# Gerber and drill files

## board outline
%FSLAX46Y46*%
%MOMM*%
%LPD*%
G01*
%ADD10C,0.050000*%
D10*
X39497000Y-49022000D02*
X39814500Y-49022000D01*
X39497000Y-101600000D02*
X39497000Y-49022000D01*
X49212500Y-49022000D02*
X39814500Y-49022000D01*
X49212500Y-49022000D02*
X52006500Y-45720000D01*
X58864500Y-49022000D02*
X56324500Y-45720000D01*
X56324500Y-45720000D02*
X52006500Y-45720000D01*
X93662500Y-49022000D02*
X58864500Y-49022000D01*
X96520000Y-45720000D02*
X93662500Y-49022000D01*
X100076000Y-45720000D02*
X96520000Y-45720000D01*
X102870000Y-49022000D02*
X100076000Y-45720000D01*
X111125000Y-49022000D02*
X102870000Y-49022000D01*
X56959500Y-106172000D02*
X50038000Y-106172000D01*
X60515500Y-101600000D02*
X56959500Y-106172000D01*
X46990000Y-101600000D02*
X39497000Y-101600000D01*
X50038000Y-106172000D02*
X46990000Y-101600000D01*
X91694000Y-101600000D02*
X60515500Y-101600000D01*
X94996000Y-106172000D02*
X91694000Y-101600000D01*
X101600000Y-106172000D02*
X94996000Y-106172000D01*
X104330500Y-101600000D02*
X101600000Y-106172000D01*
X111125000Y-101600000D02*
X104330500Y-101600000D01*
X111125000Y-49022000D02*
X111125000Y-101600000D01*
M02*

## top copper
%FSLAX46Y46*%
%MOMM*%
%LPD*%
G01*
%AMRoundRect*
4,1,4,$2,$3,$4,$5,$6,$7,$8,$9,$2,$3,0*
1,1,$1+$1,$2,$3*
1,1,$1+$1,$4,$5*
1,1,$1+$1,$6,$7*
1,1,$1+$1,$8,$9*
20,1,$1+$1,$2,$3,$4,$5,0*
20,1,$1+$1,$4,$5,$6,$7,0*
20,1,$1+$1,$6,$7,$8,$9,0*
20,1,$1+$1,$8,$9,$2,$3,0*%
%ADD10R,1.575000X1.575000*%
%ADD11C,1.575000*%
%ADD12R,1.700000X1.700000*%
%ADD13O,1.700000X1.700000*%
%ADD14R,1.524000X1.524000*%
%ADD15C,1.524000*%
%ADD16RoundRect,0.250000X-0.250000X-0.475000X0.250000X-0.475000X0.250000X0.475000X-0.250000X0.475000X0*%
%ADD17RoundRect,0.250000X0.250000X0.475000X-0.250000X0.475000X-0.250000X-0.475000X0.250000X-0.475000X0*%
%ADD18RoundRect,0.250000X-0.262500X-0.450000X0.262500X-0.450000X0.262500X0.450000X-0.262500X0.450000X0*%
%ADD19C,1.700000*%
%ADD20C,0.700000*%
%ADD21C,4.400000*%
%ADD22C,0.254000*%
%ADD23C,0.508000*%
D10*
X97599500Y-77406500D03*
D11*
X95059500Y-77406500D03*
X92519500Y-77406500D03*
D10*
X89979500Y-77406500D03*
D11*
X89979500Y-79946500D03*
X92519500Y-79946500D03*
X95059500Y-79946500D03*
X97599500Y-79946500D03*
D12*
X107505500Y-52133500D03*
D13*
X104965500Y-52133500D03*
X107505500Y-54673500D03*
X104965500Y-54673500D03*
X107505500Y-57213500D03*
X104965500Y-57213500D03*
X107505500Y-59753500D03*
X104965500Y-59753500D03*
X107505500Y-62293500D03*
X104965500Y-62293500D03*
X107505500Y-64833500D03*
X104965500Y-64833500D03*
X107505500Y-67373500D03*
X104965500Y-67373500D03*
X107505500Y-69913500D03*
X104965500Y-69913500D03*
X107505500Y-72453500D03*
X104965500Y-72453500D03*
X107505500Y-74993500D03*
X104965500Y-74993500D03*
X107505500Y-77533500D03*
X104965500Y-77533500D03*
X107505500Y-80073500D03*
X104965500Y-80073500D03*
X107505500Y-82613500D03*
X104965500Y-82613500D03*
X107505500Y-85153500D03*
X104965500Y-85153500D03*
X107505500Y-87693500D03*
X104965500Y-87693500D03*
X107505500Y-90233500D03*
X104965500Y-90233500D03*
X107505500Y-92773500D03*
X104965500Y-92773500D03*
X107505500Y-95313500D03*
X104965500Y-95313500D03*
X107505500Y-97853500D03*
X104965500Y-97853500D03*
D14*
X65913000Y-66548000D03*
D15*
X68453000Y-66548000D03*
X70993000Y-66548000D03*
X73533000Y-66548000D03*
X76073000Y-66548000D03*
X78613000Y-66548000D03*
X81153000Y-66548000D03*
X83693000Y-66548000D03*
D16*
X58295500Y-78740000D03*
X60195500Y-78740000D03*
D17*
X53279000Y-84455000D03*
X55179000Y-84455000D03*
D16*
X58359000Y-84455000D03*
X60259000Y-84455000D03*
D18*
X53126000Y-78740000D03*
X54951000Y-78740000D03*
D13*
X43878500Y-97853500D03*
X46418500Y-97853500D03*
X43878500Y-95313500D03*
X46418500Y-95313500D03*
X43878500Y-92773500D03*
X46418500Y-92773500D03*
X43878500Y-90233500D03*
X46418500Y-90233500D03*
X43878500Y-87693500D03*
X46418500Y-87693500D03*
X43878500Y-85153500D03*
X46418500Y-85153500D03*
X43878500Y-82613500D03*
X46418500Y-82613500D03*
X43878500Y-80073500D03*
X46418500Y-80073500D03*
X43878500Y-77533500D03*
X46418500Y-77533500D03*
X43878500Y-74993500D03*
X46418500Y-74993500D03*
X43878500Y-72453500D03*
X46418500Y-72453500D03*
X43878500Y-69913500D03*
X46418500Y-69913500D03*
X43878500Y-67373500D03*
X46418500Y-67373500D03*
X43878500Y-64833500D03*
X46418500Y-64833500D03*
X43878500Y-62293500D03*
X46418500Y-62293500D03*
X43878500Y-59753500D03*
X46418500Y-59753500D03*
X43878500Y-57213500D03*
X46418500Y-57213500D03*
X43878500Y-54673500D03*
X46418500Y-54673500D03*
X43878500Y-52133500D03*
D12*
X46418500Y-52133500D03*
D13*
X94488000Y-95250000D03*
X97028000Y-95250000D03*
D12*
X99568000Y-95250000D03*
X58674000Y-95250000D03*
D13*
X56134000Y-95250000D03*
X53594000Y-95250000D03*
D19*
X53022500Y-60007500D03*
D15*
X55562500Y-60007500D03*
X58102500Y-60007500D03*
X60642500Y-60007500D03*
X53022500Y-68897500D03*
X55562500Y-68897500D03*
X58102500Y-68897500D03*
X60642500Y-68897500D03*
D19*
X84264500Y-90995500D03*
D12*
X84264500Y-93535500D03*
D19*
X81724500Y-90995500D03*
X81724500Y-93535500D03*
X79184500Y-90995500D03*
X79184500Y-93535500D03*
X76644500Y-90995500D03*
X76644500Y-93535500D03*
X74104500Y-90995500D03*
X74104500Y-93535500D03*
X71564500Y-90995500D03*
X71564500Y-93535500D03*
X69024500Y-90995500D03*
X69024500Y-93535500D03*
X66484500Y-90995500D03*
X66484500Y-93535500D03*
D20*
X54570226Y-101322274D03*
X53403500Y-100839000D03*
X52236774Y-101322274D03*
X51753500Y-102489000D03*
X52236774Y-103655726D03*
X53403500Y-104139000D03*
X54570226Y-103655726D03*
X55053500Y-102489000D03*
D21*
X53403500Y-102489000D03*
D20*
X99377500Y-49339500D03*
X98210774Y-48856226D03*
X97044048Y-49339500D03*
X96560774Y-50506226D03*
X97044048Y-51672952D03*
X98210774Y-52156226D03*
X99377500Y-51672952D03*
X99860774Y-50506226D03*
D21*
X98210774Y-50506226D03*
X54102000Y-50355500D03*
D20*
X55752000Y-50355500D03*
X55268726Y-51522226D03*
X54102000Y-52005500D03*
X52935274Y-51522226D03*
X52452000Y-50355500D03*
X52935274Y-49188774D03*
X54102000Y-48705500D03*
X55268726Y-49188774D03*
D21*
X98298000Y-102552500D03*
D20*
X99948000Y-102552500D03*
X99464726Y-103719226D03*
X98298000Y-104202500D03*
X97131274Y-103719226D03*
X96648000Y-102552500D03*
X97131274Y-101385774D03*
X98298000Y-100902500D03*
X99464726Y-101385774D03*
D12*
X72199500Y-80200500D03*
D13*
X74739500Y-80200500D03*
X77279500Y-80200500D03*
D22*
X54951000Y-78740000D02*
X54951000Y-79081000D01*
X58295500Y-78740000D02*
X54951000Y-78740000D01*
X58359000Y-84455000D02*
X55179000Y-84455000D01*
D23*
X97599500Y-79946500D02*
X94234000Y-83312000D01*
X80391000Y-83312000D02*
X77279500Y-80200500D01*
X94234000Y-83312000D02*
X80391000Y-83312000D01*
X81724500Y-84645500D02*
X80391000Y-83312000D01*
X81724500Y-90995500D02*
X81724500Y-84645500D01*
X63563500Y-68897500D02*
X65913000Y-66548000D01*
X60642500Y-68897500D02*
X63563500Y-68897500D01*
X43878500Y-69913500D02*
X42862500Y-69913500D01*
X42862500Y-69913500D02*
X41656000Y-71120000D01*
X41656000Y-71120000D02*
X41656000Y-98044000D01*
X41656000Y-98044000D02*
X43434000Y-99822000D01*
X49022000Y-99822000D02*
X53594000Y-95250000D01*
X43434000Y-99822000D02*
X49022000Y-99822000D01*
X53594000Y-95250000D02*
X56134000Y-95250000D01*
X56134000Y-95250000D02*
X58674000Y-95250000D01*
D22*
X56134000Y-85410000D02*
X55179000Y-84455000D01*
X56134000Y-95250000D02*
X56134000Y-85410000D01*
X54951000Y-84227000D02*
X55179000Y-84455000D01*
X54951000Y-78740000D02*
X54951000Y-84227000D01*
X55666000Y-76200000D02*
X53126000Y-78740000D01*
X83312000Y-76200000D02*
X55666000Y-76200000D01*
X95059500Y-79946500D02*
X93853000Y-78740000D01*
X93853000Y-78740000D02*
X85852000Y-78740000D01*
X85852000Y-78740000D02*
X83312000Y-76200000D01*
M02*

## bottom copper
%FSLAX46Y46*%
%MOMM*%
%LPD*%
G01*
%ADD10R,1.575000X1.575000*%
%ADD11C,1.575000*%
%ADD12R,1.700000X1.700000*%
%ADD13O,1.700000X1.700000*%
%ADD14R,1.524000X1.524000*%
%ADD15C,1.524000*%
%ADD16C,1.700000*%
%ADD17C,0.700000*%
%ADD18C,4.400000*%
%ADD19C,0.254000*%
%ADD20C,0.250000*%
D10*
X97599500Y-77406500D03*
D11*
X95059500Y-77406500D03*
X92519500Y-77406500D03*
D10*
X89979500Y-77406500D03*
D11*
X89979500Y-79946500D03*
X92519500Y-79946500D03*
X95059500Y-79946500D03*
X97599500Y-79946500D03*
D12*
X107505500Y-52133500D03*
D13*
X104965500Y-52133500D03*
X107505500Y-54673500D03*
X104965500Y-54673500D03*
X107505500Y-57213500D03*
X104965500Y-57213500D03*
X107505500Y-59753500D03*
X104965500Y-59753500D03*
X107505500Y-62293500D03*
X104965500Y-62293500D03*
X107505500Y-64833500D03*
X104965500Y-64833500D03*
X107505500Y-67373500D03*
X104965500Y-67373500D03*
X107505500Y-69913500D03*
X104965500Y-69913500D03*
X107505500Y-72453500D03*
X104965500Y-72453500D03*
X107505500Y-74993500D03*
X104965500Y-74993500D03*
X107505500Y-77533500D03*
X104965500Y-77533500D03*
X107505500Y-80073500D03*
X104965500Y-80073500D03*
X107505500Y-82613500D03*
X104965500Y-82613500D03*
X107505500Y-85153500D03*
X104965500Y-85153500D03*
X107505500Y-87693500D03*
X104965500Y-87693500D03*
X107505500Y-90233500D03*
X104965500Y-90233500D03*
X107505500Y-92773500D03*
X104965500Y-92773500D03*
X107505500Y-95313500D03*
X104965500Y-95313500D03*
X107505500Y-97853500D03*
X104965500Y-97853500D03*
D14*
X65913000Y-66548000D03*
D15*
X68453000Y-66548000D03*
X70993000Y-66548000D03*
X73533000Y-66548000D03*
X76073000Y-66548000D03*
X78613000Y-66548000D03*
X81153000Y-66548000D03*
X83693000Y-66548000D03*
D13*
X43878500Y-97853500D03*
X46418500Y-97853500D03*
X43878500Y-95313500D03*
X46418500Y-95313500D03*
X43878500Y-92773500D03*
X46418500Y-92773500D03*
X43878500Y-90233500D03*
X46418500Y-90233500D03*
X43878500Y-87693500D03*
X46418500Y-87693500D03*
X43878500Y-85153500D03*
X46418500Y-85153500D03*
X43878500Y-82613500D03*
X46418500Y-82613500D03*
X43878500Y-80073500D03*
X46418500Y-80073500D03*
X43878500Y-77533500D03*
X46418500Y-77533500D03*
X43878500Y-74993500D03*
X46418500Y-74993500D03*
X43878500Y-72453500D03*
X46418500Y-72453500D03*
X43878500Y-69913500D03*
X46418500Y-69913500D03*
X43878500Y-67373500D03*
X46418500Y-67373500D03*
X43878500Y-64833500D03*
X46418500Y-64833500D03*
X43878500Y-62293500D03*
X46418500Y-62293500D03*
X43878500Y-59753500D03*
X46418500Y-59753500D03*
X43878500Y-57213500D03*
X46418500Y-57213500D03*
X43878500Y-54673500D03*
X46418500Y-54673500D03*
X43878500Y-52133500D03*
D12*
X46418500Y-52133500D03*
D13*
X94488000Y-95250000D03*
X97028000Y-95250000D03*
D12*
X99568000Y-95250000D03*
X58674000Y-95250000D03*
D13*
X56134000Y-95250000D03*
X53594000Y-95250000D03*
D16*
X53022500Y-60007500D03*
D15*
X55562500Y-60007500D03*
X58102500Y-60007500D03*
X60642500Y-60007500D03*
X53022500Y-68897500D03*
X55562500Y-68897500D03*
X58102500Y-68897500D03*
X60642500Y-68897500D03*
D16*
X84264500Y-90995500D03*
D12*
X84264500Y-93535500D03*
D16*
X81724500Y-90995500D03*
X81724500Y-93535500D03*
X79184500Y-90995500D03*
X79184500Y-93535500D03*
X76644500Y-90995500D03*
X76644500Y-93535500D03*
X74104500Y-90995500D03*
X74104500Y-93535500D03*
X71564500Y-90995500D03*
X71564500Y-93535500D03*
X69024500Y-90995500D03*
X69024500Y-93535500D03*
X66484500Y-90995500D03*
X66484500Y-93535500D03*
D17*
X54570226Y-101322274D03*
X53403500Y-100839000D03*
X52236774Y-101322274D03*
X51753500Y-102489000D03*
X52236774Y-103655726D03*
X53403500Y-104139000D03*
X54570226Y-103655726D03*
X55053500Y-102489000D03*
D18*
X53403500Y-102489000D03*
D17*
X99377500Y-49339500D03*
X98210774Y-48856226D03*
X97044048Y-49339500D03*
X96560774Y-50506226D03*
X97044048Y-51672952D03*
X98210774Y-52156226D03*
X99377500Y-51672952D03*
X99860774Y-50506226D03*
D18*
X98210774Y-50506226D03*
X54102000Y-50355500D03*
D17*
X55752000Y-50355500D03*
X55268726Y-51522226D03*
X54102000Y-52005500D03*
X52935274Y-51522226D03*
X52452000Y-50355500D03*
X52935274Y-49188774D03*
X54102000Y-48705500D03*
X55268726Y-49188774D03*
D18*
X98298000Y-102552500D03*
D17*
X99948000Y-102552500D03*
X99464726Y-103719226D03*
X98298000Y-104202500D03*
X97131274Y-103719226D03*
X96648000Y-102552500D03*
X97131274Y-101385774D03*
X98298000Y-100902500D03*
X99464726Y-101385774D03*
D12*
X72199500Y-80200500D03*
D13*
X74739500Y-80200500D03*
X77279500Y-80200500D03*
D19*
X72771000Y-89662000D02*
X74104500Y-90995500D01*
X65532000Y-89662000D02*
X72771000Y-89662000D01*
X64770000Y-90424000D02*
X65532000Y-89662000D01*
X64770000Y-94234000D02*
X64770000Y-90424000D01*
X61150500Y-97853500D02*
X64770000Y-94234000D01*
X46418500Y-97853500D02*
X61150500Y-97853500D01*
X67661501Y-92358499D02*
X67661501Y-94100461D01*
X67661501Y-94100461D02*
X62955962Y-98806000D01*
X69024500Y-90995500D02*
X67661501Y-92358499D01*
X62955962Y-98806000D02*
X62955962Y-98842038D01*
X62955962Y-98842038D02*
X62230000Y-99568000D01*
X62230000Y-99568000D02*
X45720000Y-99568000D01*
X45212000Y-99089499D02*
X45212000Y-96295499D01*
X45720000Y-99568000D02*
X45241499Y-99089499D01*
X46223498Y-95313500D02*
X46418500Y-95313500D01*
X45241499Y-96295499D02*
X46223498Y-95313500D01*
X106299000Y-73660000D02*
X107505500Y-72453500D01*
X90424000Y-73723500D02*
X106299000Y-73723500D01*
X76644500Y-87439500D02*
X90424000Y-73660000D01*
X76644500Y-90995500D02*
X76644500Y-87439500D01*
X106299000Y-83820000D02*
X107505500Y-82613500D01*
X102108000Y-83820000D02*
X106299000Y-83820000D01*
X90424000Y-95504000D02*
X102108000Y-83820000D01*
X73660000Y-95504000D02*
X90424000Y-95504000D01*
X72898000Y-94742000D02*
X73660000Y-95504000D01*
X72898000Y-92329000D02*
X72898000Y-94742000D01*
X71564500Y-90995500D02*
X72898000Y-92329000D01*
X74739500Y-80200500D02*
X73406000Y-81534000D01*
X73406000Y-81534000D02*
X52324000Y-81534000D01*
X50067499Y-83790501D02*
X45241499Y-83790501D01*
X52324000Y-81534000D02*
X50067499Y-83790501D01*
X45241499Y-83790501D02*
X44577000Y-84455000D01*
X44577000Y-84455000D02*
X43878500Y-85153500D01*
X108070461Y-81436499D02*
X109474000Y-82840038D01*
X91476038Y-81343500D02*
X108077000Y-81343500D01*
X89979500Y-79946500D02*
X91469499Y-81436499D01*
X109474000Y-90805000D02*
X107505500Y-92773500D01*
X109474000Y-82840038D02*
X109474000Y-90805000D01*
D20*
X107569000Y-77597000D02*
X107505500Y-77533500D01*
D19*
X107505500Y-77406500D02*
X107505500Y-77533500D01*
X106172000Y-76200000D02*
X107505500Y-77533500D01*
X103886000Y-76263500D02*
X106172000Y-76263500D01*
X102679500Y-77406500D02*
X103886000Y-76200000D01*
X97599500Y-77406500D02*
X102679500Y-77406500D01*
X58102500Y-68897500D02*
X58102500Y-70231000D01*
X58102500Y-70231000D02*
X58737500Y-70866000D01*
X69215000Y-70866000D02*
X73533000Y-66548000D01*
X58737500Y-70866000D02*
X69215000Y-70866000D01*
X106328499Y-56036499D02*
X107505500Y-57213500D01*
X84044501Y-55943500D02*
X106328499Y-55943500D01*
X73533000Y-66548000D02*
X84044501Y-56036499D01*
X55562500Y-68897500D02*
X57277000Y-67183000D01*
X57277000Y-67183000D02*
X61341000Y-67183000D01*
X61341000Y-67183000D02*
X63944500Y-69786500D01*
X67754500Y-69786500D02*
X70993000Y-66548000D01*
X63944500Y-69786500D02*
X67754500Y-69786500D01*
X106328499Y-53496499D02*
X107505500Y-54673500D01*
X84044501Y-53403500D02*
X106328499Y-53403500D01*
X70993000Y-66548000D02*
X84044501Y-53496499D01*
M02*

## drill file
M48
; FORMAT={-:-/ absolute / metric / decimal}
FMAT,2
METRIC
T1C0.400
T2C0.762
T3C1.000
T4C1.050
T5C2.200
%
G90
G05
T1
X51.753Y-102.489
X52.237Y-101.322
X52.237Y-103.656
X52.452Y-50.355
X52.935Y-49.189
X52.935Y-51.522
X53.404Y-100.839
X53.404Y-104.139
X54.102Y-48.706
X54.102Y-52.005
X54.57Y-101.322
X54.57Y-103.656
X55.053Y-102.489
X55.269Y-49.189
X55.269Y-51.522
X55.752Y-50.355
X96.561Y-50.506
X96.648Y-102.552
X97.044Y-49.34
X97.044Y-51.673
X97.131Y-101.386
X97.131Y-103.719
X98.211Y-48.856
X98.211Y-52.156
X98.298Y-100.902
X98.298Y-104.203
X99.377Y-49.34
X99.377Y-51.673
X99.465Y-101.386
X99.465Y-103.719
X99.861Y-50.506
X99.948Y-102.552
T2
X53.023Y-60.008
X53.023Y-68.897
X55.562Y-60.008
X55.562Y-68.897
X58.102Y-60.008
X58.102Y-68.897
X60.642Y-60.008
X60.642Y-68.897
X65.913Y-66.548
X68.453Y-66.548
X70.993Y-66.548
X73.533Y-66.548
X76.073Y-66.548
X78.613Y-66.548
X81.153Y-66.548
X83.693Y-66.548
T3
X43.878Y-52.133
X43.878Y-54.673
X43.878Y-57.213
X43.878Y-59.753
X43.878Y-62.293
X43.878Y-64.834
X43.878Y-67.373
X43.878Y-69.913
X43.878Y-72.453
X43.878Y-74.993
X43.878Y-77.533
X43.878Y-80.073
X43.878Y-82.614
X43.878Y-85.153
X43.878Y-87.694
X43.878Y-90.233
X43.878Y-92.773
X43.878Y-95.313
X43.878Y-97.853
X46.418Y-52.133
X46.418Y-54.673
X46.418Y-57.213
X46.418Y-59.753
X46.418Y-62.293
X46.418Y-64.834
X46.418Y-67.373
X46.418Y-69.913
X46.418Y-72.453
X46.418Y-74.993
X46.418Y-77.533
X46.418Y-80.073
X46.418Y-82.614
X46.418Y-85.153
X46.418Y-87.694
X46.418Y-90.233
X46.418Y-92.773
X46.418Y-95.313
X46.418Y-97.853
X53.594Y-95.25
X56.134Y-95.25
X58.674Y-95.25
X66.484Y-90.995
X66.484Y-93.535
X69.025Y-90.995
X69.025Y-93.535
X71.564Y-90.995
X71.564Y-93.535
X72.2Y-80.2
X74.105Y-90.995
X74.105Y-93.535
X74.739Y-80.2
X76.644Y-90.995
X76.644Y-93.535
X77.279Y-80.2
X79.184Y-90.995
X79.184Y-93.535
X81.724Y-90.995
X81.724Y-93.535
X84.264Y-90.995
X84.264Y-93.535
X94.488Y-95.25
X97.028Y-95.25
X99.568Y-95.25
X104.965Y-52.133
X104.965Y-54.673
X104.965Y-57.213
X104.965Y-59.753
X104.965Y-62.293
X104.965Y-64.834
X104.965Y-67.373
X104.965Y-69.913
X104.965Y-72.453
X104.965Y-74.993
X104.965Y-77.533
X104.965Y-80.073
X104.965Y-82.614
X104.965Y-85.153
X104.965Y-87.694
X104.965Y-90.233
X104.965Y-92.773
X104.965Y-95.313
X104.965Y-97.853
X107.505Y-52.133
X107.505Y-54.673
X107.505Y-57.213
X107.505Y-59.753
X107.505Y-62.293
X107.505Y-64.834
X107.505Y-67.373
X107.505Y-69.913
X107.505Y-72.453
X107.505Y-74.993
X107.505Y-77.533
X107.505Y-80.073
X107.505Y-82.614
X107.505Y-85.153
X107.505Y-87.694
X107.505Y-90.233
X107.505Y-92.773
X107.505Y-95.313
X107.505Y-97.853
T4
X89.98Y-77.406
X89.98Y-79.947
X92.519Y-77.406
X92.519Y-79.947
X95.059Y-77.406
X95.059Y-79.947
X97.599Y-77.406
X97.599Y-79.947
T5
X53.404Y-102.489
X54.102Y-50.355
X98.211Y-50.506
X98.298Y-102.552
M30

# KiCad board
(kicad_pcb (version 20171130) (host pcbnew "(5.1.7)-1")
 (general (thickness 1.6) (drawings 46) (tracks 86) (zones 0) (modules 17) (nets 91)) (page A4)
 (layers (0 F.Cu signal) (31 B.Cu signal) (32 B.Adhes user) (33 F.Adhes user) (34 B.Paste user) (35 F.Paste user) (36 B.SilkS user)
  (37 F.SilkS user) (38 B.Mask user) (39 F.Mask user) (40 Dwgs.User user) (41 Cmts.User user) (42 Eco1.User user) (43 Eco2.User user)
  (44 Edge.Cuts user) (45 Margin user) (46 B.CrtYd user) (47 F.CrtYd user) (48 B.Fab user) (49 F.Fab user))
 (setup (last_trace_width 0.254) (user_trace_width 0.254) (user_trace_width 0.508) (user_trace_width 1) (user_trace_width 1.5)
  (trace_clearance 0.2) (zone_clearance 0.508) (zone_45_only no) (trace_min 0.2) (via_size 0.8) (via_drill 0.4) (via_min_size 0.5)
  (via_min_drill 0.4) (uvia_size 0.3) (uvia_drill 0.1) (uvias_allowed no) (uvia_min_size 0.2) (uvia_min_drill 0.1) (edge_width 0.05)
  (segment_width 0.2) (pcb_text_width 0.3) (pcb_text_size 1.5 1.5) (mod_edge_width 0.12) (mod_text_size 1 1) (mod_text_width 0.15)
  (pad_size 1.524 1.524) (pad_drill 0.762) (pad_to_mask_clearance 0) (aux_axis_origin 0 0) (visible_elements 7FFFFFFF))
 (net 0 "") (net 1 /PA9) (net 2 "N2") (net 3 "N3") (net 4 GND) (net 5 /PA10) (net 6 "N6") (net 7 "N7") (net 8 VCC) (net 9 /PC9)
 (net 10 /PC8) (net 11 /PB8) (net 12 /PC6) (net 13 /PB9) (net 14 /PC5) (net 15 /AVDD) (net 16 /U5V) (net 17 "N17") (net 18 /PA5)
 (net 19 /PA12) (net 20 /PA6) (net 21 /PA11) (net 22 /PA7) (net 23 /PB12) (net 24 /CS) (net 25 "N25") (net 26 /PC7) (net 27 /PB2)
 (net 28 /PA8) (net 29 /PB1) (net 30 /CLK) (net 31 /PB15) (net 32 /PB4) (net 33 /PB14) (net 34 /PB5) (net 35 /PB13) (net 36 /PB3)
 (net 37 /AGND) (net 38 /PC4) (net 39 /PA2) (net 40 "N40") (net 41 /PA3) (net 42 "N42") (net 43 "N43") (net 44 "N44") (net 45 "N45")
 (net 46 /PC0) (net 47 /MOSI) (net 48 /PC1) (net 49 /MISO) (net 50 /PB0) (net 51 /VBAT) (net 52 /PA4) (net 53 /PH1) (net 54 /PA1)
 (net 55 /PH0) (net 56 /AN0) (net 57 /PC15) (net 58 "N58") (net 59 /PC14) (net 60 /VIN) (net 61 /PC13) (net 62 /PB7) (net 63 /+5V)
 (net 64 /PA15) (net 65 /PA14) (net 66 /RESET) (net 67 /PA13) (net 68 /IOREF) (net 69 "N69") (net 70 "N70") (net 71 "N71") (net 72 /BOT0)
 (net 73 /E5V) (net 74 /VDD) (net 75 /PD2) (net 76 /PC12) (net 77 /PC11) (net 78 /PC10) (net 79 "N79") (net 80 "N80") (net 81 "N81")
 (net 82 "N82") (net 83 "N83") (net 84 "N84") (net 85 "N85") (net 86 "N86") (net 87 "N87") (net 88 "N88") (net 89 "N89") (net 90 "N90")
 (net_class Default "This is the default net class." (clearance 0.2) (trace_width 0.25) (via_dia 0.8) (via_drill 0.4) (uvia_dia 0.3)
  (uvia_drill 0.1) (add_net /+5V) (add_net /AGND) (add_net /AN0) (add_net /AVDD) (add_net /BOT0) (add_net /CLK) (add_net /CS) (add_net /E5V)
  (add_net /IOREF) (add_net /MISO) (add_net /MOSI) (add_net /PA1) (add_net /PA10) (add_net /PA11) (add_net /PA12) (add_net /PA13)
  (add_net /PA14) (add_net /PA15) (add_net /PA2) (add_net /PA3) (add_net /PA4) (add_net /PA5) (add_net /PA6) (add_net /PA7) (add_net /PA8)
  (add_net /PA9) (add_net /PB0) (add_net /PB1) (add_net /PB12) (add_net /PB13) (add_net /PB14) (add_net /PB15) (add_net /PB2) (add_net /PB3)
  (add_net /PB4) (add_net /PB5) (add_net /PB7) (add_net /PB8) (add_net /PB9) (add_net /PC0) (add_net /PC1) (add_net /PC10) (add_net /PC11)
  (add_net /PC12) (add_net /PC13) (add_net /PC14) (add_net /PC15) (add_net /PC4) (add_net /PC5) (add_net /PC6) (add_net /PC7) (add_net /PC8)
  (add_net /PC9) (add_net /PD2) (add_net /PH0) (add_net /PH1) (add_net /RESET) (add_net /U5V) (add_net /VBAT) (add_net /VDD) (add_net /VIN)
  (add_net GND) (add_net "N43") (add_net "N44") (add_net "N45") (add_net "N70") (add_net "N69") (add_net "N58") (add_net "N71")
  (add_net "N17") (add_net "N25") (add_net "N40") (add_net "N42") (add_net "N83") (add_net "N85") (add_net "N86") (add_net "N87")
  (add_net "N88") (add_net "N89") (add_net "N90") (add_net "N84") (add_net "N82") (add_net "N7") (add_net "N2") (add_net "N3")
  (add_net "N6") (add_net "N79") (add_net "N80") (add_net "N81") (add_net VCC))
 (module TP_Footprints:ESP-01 (layer F.Cu) (at 93.7895 77.4065 90)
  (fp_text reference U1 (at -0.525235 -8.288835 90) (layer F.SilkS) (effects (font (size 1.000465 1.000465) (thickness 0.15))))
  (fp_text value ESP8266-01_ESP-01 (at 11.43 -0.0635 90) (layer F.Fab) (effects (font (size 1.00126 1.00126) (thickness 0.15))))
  (pad 1 thru_hole rect (at 0 3.81 90) (size 1.575 1.575) (drill 1.05) (layers *.Cu *.Mask) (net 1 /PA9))
  (pad 2 thru_hole circle (at 0 1.27 90) (size 1.575 1.575) (drill 1.05) (layers *.Cu *.Mask) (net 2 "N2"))
  (pad 3 thru_hole circle (at 0 -1.27 90) (size 1.575 1.575) (drill 1.05) (layers *.Cu *.Mask) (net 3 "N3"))
  (pad 4 thru_hole rect (at 0 -3.81 90) (size 1.575 1.575) (drill 1.05) (layers *.Cu *.Mask) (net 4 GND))
  (pad 5 thru_hole circle (at -2.54 -3.81 90) (size 1.575 1.575) (drill 1.05) (layers *.Cu *.Mask) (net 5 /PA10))
  (pad 6 thru_hole circle (at -2.54 -1.27 90) (size 1.575 1.575) (drill 1.05) (layers *.Cu *.Mask) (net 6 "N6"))
  (pad 7 thru_hole circle (at -2.54 1.27 90) (size 1.575 1.575) (drill 1.05) (layers *.Cu *.Mask) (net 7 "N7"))
  (pad 8 thru_hole circle (at -2.54 3.81 90) (size 1.575 1.575) (drill 1.05) (layers *.Cu *.Mask) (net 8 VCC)))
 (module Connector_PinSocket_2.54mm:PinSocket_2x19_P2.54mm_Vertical (layer F.Cu) (at 107.5055 52.1335)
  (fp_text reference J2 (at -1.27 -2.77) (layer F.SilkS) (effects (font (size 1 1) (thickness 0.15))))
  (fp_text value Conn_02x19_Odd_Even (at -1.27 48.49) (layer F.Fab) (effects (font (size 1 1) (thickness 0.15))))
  (pad 1 thru_hole rect (at 0 0) (size 1.7 1.7) (drill 1) (layers *.Cu *.Mask) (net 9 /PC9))
  (pad 2 thru_hole oval (at -2.54 0) (size 1.7 1.7) (drill 1) (layers *.Cu *.Mask) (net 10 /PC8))
  (pad 3 thru_hole oval (at 0 2.54) (size 1.7 1.7) (drill 1) (layers *.Cu *.Mask) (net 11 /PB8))
  (pad 4 thru_hole oval (at -2.54 2.54) (size 1.7 1.7) (drill 1) (layers *.Cu *.Mask) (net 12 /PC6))
  (pad 5 thru_hole oval (at 0 5.08) (size 1.7 1.7) (drill 1) (layers *.Cu *.Mask) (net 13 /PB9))
  (pad 6 thru_hole oval (at -2.54 5.08) (size 1.7 1.7) (drill 1) (layers *.Cu *.Mask) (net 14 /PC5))
  (pad 7 thru_hole oval (at 0 7.62) (size 1.7 1.7) (drill 1) (layers *.Cu *.Mask) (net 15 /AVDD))
  (pad 8 thru_hole oval (at -2.54 7.62) (size 1.7 1.7) (drill 1) (layers *.Cu *.Mask) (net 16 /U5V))
  (pad 9 thru_hole oval (at 0 10.16) (size 1.7 1.7) (drill 1) (layers *.Cu *.Mask) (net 4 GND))
  (pad 10 thru_hole oval (at -2.54 10.16) (size 1.7 1.7) (drill 1) (layers *.Cu *.Mask) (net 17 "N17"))
  (pad 11 thru_hole oval (at 0 12.7) (size 1.7 1.7) (drill 1) (layers *.Cu *.Mask) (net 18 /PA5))
  (pad 12 thru_hole oval (at -2.54 12.7) (size 1.7 1.7) (drill 1) (layers *.Cu *.Mask) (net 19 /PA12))
  (pad 13 thru_hole oval (at 0 15.24) (size 1.7 1.7) (drill 1) (layers *.Cu *.Mask) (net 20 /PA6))
  (pad 14 thru_hole oval (at -2.54 15.24) (size 1.7 1.7) (drill 1) (layers *.Cu *.Mask) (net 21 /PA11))
  (pad 15 thru_hole oval (at 0 17.78) (size 1.7 1.7) (drill 1) (layers *.Cu *.Mask) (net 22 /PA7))
  (pad 16 thru_hole oval (at -2.54 17.78) (size 1.7 1.7) (drill 1) (layers *.Cu *.Mask) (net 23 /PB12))
  (pad 17 thru_hole oval (at 0 20.32) (size 1.7 1.7) (drill 1) (layers *.Cu *.Mask) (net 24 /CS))
  (pad 18 thru_hole oval (at -2.54 20.32) (size 1.7 1.7) (drill 1) (layers *.Cu *.Mask) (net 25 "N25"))
  (pad 19 thru_hole oval (at 0 22.86) (size 1.7 1.7) (drill 1) (layers *.Cu *.Mask) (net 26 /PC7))
  (pad 20 thru_hole oval (at -2.54 22.86) (size 1.7 1.7) (drill 1) (layers *.Cu *.Mask) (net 4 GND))
  (pad 21 thru_hole oval (at 0 25.4) (size 1.7 1.7) (drill 1) (layers *.Cu *.Mask) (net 1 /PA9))
  (pad 22 thru_hole oval (at -2.54 25.4) (size 1.7 1.7) (drill 1) (layers *.Cu *.Mask) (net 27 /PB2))
  (pad 23 thru_hole oval (at 0 27.94) (size 1.7 1.7) (drill 1) (layers *.Cu *.Mask) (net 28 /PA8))
  (pad 24 thru_hole oval (at -2.54 27.94) (size 1.7 1.7) (drill 1) (layers *.Cu *.Mask) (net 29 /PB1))
  (pad 25 thru_hole oval (at 0 30.48) (size 1.7 1.7) (drill 1) (layers *.Cu *.Mask) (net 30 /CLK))
  (pad 26 thru_hole oval (at -2.54 30.48) (size 1.7 1.7) (drill 1) (layers *.Cu *.Mask) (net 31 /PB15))
  (pad 27 thru_hole oval (at 0 33.02) (size 1.7 1.7) (drill 1) (layers *.Cu *.Mask) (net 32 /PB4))
  (pad 28 thru_hole oval (at -2.54 33.02) (size 1.7 1.7) (drill 1) (layers *.Cu *.Mask) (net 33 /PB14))
  (pad 29 thru_hole oval (at 0 35.56) (size 1.7 1.7) (drill 1) (layers *.Cu *.Mask) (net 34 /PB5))
  (pad 30 thru_hole oval (at -2.54 35.56) (size 1.7 1.7) (drill 1) (layers *.Cu *.Mask) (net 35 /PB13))
  (pad 31 thru_hole oval (at 0 38.1) (size 1.7 1.7) (drill 1) (layers *.Cu *.Mask) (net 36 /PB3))
  (pad 32 thru_hole oval (at -2.54 38.1) (size 1.7 1.7) (drill 1) (layers *.Cu *.Mask) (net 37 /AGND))
  (pad 33 thru_hole oval (at 0 40.64) (size 1.7 1.7) (drill 1) (layers *.Cu *.Mask) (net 5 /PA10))
  (pad 34 thru_hole oval (at -2.54 40.64) (size 1.7 1.7) (drill 1) (layers *.Cu *.Mask) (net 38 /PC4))
  (pad 35 thru_hole oval (at 0 43.18) (size 1.7 1.7) (drill 1) (layers *.Cu *.Mask) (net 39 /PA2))
  (pad 36 thru_hole oval (at -2.54 43.18) (size 1.7 1.7) (drill 1) (layers *.Cu *.Mask) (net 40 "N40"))
  (pad 37 thru_hole oval (at 0 45.72) (size 1.7 1.7) (drill 1) (layers *.Cu *.Mask) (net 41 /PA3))
  (pad 38 thru_hole oval (at -2.54 45.72) (size 1.7 1.7) (drill 1) (layers *.Cu *.Mask) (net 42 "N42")))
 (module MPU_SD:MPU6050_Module (layer F.Cu) (at 65.913 66.548 90)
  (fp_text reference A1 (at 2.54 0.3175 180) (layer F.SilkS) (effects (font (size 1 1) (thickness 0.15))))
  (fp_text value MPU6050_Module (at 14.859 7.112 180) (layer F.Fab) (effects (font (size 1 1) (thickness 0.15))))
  (pad 1 thru_hole rect (at 0 0 90) (size 1.524 1.524) (drill 0.762) (layers *.Cu *.Mask) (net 8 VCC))
  (pad 2 thru_hole circle (at 0 2.54 90) (size 1.524 1.524) (drill 0.762) (layers *.Cu *.Mask) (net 4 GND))
  (pad 3 thru_hole circle (at 0 5.08 90) (size 1.524 1.524) (drill 0.762) (layers *.Cu *.Mask) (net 11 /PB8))
  (pad 4 thru_hole circle (at 0 7.62 90) (size 1.524 1.524) (drill 0.762) (layers *.Cu *.Mask) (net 13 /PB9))
  (pad 5 thru_hole circle (at 0 10.16 90) (size 1.524 1.524) (drill 0.762) (layers *.Cu *.Mask) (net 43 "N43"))
  (pad 6 thru_hole circle (at 0 12.7 90) (size 1.524 1.524) (drill 0.762) (layers *.Cu *.Mask) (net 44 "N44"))
  (pad 7 thru_hole circle (at 0 15.24 90) (size 1.524 1.524) (drill 0.762) (layers *.Cu *.Mask) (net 4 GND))
  (pad 8 thru_hole circle (at 0 17.78 90) (size 1.524 1.524) (drill 0.762) (layers *.Cu *.Mask) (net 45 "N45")))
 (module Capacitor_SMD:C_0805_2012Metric (layer F.Cu) (at 59.2455 78.74)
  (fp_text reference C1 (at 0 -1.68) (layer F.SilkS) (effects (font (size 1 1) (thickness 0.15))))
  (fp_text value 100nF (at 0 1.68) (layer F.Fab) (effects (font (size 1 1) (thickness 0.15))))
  (pad 1 smd roundrect (at -0.95 0) (size 1 1.45) (layers F.Cu F.Paste F.Mask) (roundrect_rratio 0.25) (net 8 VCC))
  (pad 2 smd roundrect (at 0.95 0) (size 1 1.45) (layers F.Cu F.Paste F.Mask) (roundrect_rratio 0.25) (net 4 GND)))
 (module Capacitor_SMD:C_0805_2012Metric (layer F.Cu) (at 54.229 84.455 180)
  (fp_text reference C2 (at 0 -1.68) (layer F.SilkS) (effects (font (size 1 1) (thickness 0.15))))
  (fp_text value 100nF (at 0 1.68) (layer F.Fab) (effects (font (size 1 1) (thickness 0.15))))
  (pad 2 smd roundrect (at 0.95 0 180) (size 1 1.45) (layers F.Cu F.Paste F.Mask) (roundrect_rratio 0.25) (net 4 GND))
  (pad 1 smd roundrect (at -0.95 0 180) (size 1 1.45) (layers F.Cu F.Paste F.Mask) (roundrect_rratio 0.25) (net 8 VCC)))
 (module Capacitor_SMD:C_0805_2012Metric (layer F.Cu) (at 59.309 84.455)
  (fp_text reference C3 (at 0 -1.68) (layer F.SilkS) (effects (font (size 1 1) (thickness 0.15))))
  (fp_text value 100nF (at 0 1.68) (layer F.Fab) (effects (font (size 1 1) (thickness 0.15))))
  (pad 1 smd roundrect (at -0.95 0) (size 1 1.45) (layers F.Cu F.Paste F.Mask) (roundrect_rratio 0.25) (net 8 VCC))
  (pad 2 smd roundrect (at 0.95 0) (size 1 1.45) (layers F.Cu F.Paste F.Mask) (roundrect_rratio 0.25) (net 4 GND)))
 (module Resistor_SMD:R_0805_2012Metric (layer F.Cu) (at 54.0385 78.74)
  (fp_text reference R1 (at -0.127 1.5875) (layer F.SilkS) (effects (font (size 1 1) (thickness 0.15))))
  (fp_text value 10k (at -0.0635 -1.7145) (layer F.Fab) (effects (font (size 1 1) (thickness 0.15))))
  (pad 1 smd roundrect (at -0.9125 0) (size 1.025 1.4) (layers F.Cu F.Paste F.Mask) (roundrect_rratio 0.243902) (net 7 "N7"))
  (pad 2 smd roundrect (at 0.9125 0) (size 1.025 1.4) (layers F.Cu F.Paste F.Mask) (roundrect_rratio 0.243902) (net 8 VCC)))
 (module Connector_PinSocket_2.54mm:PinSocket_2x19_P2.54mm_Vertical (layer F.Cu) (at 46.4185 52.1335)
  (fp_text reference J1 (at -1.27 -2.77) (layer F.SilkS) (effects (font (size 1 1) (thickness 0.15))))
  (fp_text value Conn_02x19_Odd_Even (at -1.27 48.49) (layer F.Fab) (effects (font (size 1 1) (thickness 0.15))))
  (pad 38 thru_hole oval (at -2.54 45.72) (size 1.7 1.7) (drill 1) (layers *.Cu *.Mask) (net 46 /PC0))
  (pad 37 thru_hole oval (at 0 45.72) (size 1.7 1.7) (drill 1) (layers *.Cu *.Mask) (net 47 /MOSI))
  (pad 36 thru_hole oval (at -2.54 43.18) (size 1.7 1.7) (drill 1) (layers *.Cu *.Mask) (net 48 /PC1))
  (pad 35 thru_hole oval (at 0 43.18) (size 1.7 1.7) (drill 1) (layers *.Cu *.Mask) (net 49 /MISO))
  (pad 34 thru_hole oval (at -2.54 40.64) (size 1.7 1.7) (drill 1) (layers *.Cu *.Mask) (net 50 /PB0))
  (pad 33 thru_hole oval (at 0 40.64) (size 1.7 1.7) (drill 1) (layers *.Cu *.Mask) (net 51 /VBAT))
  (pad 32 thru_hole oval (at -2.54 38.1) (size 1.7 1.7) (drill 1) (layers *.Cu *.Mask) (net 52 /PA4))
  (pad 31 thru_hole oval (at 0 38.1) (size 1.7 1.7) (drill 1) (layers *.Cu *.Mask) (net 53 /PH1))
  (pad 30 thru_hole oval (at -2.54 35.56) (size 1.7 1.7) (drill 1) (layers *.Cu *.Mask) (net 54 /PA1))
  (pad 29 thru_hole oval (at 0 35.56) (size 1.7 1.7) (drill 1) (layers *.Cu *.Mask) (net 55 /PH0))
  (pad 28 thru_hole oval (at -2.54 33.02) (size 1.7 1.7) (drill 1) (layers *.Cu *.Mask) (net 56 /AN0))
  (pad 27 thru_hole oval (at 0 33.02) (size 1.7 1.7) (drill 1) (layers *.Cu *.Mask) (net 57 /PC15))
  (pad 26 thru_hole oval (at -2.54 30.48) (size 1.7 1.7) (drill 1) (layers *.Cu *.Mask) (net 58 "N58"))
  (pad 25 thru_hole oval (at 0 30.48) (size 1.7 1.7) (drill 1) (layers *.Cu *.Mask) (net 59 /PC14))
  (pad 24 thru_hole oval (at -2.54 27.94) (size 1.7 1.7) (drill 1) (layers *.Cu *.Mask) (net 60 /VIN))
  (pad 23 thru_hole oval (at 0 27.94) (size 1.7 1.7) (drill 1) (layers *.Cu *.Mask) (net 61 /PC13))
  (pad 22 thru_hole oval (at -2.54 25.4) (size 1.7 1.7) (drill 1) (layers *.Cu *.Mask) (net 4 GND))
  (pad 21 thru_hole oval (at 0 25.4) (size 1.7 1.7) (drill 1) (layers *.Cu *.Mask) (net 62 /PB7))
  (pad 20 thru_hole oval (at -2.54 22.86) (size 1.7 1.7) (drill 1) (layers *.Cu *.Mask) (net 4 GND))
  (pad 19 thru_hole oval (at 0 22.86) (size 1.7 1.7) (drill 1) (layers *.Cu *.Mask) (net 4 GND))
  (pad 18 thru_hole oval (at -2.54 20.32) (size 1.7 1.7) (drill 1) (layers *.Cu *.Mask) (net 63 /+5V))
  (pad 17 thru_hole oval (at 0 20.32) (size 1.7 1.7) (drill 1) (layers *.Cu *.Mask) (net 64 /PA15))
  (pad 16 thru_hole oval (at -2.54 17.78) (size 1.7 1.7) (drill 1) (layers *.Cu *.Mask) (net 8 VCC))
  (pad 15 thru_hole oval (at 0 17.78) (size 1.7 1.7) (drill 1) (layers *.Cu *.Mask) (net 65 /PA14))
  (pad 14 thru_hole oval (at -2.54 15.24) (size 1.7 1.7) (drill 1) (layers *.Cu *.Mask) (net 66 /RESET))
  (pad 13 thru_hole oval (at 0 15.24) (size 1.7 1.7) (drill 1) (layers *.Cu *.Mask) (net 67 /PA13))
  (pad 12 thru_hole oval (at -2.54 12.7) (size 1.7 1.7) (drill 1) (layers *.Cu *.Mask) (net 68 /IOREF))
  (pad 11 thru_hole oval (at 0 12.7) (size 1.7 1.7) (drill 1) (layers *.Cu *.Mask) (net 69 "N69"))
  (pad 10 thru_hole oval (at -2.54 10.16) (size 1.7 1.7) (drill 1) (layers *.Cu *.Mask) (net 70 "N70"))
  (pad 9 thru_hole oval (at 0 10.16) (size 1.7 1.7) (drill 1) (layers *.Cu *.Mask) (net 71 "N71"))
  (pad 8 thru_hole oval (at -2.54 7.62) (size 1.7 1.7) (drill 1) (layers *.Cu *.Mask) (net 4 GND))
  (pad 7 thru_hole oval (at 0 7.62) (size 1.7 1.7) (drill 1) (layers *.Cu *.Mask) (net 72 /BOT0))
  (pad 6 thru_hole oval (at -2.54 5.08) (size 1.7 1.7) (drill 1) (layers *.Cu *.Mask) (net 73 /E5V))
  (pad 5 thru_hole oval (at 0 5.08) (size 1.7 1.7) (drill 1) (layers *.Cu *.Mask) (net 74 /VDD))
  (pad 4 thru_hole oval (at -2.54 2.54) (size 1.7 1.7) (drill 1) (layers *.Cu *.Mask) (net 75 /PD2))
  (pad 3 thru_hole oval (at 0 2.54) (size 1.7 1.7) (drill 1) (layers *.Cu *.Mask) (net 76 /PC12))
  (pad 2 thru_hole oval (at -2.54 0) (size 1.7 1.7) (drill 1) (layers *.Cu *.Mask) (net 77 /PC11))
  (pad 1 thru_hole rect (at 0 0) (size 1.7 1.7) (drill 1) (layers *.Cu *.Mask) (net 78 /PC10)))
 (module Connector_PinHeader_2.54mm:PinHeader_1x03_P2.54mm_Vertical (layer F.Cu) (at 99.568 95.25 270)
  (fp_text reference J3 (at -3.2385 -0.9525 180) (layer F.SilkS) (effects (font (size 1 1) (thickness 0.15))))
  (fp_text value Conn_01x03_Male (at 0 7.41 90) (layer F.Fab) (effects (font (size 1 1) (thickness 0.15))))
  (pad 3 thru_hole oval (at 0 5.08 270) (size 1.7 1.7) (drill 1) (layers *.Cu *.Mask) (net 4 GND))
  (pad 2 thru_hole oval (at 0 2.54 270) (size 1.7 1.7) (drill 1) (layers *.Cu *.Mask) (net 4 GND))
  (pad 1 thru_hole rect (at 0 0 270) (size 1.7 1.7) (drill 1) (layers *.Cu *.Mask) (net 4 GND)))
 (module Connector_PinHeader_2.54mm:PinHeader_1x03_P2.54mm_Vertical (layer F.Cu) (at 58.674 95.25 270)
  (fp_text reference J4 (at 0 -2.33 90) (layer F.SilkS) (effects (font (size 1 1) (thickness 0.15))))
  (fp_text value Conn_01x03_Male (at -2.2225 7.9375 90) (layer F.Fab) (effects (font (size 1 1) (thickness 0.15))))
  (pad 1 thru_hole rect (at 0 0 270) (size 1.7 1.7) (drill 1) (layers *.Cu *.Mask) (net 8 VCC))
  (pad 2 thru_hole oval (at 0 2.54 270) (size 1.7 1.7) (drill 1) (layers *.Cu *.Mask) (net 8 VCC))
  (pad 3 thru_hole oval (at 0 5.08 270) (size 1.7 1.7) (drill 1) (layers *.Cu *.Mask) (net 8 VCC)))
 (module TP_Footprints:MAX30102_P (layer F.Cu) (at 55.5625 60.0075)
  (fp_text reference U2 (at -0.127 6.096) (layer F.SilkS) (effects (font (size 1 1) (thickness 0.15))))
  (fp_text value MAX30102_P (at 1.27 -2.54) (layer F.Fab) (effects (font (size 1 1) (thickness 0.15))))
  (pad 1 thru_hole circle (at -2.54 0) (size 1.7 1.7) (drill 0.762) (layers *.Cu *.Mask) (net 4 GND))
  (pad 2 thru_hole circle (at 0 0) (size 1.524 1.524) (drill 0.762) (layers *.Cu *.Mask) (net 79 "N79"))
  (pad 3 thru_hole circle (at 2.54 0) (size 1.524 1.524) (drill 0.762) (layers *.Cu *.Mask) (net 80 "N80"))
  (pad 4 thru_hole circle (at 5.08 0) (size 1.524 1.524) (drill 0.762) (layers *.Cu *.Mask) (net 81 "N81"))
  (pad 5 thru_hole circle (at -2.54 8.89) (size 1.524 1.524) (drill 0.762) (layers *.Cu *.Mask) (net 4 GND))
  (pad 6 thru_hole circle (at 0 8.89) (size 1.524 1.524) (drill 0.762) (layers *.Cu *.Mask) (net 11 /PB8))
  (pad 7 thru_hole circle (at 2.54 8.89) (size 1.524 1.524) (drill 0.762) (layers *.Cu *.Mask) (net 13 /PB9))
  (pad 8 thru_hole circle (at 5.08 8.89) (size 1.524 1.524) (drill 0.762) (layers *.Cu *.Mask) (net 8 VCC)))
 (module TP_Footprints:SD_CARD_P (layer F.Cu) (at 84.2645 93.5355 270)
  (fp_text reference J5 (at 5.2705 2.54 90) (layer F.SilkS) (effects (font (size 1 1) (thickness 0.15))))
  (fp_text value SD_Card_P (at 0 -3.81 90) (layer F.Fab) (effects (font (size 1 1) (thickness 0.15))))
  (pad 1 thru_hole circle (at -2.54 0 270) (size 1.7 1.7) (drill 1) (layers *.Cu *.Mask) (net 4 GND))
  (pad 9 thru_hole rect (at 0 0 270) (size 1.7 1.7) (drill 1) (layers *.Cu *.Mask) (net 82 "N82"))
  (pad 2 thru_hole circle (at -2.54 2.54 270) (size 1.7 1.7) (drill 1) (layers *.Cu *.Mask) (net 8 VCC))
  (pad 10 thru_hole circle (at 0 2.54 270) (size 1.7 1.7) (drill 1) (layers *.Cu *.Mask) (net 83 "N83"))
  (pad 3 thru_hole circle (at -2.54 5.08 270) (size 1.7 1.7) (drill 1) (layers *.Cu *.Mask) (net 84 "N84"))
  (pad 11 thru_hole circle (at 0 5.08 270) (size 1.7 1.7) (drill 1) (layers *.Cu *.Mask) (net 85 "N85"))
  (pad 4 thru_hole circle (at -2.54 7.62 270) (size 1.7 1.7) (drill 1) (layers *.Cu *.Mask) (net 24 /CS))
  (pad 12 thru_hole circle (at 0 7.62 270) (size 1.7 1.7) (drill 1) (layers *.Cu *.Mask) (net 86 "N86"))
  (pad 5 thru_hole circle (at -2.54 10.16 270) (size 1.7 1.7) (drill 1) (layers *.Cu *.Mask) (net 47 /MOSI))
  (pad 13 thru_hole circle (at 0 10.16 270) (size 1.7 1.7) (drill 1) (layers *.Cu *.Mask) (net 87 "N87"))
  (pad 6 thru_hole circle (at -2.54 12.7 270) (size 1.7 1.7) (drill 1) (layers *.Cu *.Mask) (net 30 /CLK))
  (pad 14 thru_hole circle (at 0 12.7 270) (size 1.7 1.7) (drill 1) (layers *.Cu *.Mask) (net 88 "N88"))
  (pad 7 thru_hole circle (at -2.54 15.24 270) (size 1.7 1.7) (drill 1) (layers *.Cu *.Mask) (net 49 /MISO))
  (pad 15 thru_hole circle (at 0 15.24 270) (size 1.7 1.7) (drill 1) (layers *.Cu *.Mask) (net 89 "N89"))
  (pad 8 thru_hole circle (at -2.54 17.78 270) (size 1.7 1.7) (drill 1) (layers *.Cu *.Mask) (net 4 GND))
  (pad 16 thru_hole circle (at 0 17.78 270) (size 1.7 1.7) (drill 1) (layers *.Cu *.Mask) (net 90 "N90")))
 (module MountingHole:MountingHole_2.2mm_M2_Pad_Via (layer F.Cu) (at 53.4035 102.489)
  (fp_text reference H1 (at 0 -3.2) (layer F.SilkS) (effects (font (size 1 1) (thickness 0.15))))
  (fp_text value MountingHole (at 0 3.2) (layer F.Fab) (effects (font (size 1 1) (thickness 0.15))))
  (pad 1 thru_hole circle (at 1.166726 -1.166726) (size 0.7 0.7) (drill 0.4) (layers *.Cu *.Mask))
  (pad 1 thru_hole circle (at 0 -1.65) (size 0.7 0.7) (drill 0.4) (layers *.Cu *.Mask))
  (pad 1 thru_hole circle (at -1.166726 -1.166726) (size 0.7 0.7) (drill 0.4) (layers *.Cu *.Mask))
  (pad 1 thru_hole circle (at -1.65 0) (size 0.7 0.7) (drill 0.4) (layers *.Cu *.Mask))
  (pad 1 thru_hole circle (at -1.166726 1.166726) (size 0.7 0.7) (drill 0.4) (layers *.Cu *.Mask))
  (pad 1 thru_hole circle (at 0 1.65) (size 0.7 0.7) (drill 0.4) (layers *.Cu *.Mask))
  (pad 1 thru_hole circle (at 1.166726 1.166726) (size 0.7 0.7) (drill 0.4) (layers *.Cu *.Mask))
  (pad 1 thru_hole circle (at 1.65 0) (size 0.7 0.7) (drill 0.4) (layers *.Cu *.Mask))
  (pad 1 thru_hole circle (at 0 0) (size 4.4 4.4) (drill 2.2) (layers *.Cu *.Mask)))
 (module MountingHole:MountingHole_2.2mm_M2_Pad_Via (layer F.Cu) (at 98.210774 50.506226)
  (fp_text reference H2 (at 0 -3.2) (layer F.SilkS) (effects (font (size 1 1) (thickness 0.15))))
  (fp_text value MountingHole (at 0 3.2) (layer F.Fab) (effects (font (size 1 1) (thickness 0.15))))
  (pad 1 thru_hole circle (at 1.166726 -1.166726) (size 0.7 0.7) (drill 0.4) (layers *.Cu *.Mask))
  (pad 1 thru_hole circle (at 0 -1.65) (size 0.7 0.7) (drill 0.4) (layers *.Cu *.Mask))
  (pad 1 thru_hole circle (at -1.166726 -1.166726) (size 0.7 0.7) (drill 0.4) (layers *.Cu *.Mask))
  (pad 1 thru_hole circle (at -1.65 0) (size 0.7 0.7) (drill 0.4) (layers *.Cu *.Mask))
  (pad 1 thru_hole circle (at -1.166726 1.166726) (size 0.7 0.7) (drill 0.4) (layers *.Cu *.Mask))
  (pad 1 thru_hole circle (at 0 1.65) (size 0.7 0.7) (drill 0.4) (layers *.Cu *.Mask))
  (pad 1 thru_hole circle (at 1.166726 1.166726) (size 0.7 0.7) (drill 0.4) (layers *.Cu *.Mask))
  (pad 1 thru_hole circle (at 1.65 0) (size 0.7 0.7) (drill 0.4) (layers *.Cu *.Mask))
  (pad 1 thru_hole circle (at 0 0) (size 4.4 4.4) (drill 2.2) (layers *.Cu *.Mask)))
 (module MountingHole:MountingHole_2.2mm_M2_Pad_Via (layer F.Cu) (at 54.102 50.3555)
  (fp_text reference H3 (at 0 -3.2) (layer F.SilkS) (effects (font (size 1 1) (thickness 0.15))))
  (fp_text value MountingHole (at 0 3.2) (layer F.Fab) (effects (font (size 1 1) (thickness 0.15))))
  (pad 1 thru_hole circle (at 0 0) (size 4.4 4.4) (drill 2.2) (layers *.Cu *.Mask))
  (pad 1 thru_hole circle (at 1.65 0) (size 0.7 0.7) (drill 0.4) (layers *.Cu *.Mask))
  (pad 1 thru_hole circle (at 1.166726 1.166726) (size 0.7 0.7) (drill 0.4) (layers *.Cu *.Mask))
  (pad 1 thru_hole circle (at 0 1.65) (size 0.7 0.7) (drill 0.4) (layers *.Cu *.Mask))
  (pad 1 thru_hole circle (at -1.166726 1.166726) (size 0.7 0.7) (drill 0.4) (layers *.Cu *.Mask))
  (pad 1 thru_hole circle (at -1.65 0) (size 0.7 0.7) (drill 0.4) (layers *.Cu *.Mask))
  (pad 1 thru_hole circle (at -1.166726 -1.166726) (size 0.7 0.7) (drill 0.4) (layers *.Cu *.Mask))
  (pad 1 thru_hole circle (at 0 -1.65) (size 0.7 0.7) (drill 0.4) (layers *.Cu *.Mask))
  (pad 1 thru_hole circle (at 1.166726 -1.166726) (size 0.7 0.7) (drill 0.4) (layers *.Cu *.Mask)))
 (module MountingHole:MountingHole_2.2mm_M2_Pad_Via (layer F.Cu) (at 98.298 102.5525)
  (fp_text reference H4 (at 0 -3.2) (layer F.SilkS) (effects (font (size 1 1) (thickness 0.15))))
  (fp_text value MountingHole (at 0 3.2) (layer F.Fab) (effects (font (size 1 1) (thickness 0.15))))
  (pad 1 thru_hole circle (at 0 0) (size 4.4 4.4) (drill 2.2) (layers *.Cu *.Mask))
  (pad 1 thru_hole circle (at 1.65 0) (size 0.7 0.7) (drill 0.4) (layers *.Cu *.Mask))
  (pad 1 thru_hole circle (at 1.166726 1.166726) (size 0.7 0.7) (drill 0.4) (layers *.Cu *.Mask))
  (pad 1 thru_hole circle (at 0 1.65) (size 0.7 0.7) (drill 0.4) (layers *.Cu *.Mask))
  (pad 1 thru_hole circle (at -1.166726 1.166726) (size 0.7 0.7) (drill 0.4) (layers *.Cu *.Mask))
  (pad 1 thru_hole circle (at -1.65 0) (size 0.7 0.7) (drill 0.4) (layers *.Cu *.Mask))
  (pad 1 thru_hole circle (at -1.166726 -1.166726) (size 0.7 0.7) (drill 0.4) (layers *.Cu *.Mask))
  (pad 1 thru_hole circle (at 0 -1.65) (size 0.7 0.7) (drill 0.4) (layers *.Cu *.Mask))
  (pad 1 thru_hole circle (at 1.166726 -1.166726) (size 0.7 0.7) (drill 0.4) (layers *.Cu *.Mask)))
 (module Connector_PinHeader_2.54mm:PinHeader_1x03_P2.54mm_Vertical (layer F.Cu) (at 72.1995 80.2005 90)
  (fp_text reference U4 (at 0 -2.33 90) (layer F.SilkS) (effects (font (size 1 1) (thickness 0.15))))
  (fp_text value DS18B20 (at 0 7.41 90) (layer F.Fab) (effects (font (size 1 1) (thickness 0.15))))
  (pad 1 thru_hole rect (at 0 0 90) (size 1.7 1.7) (drill 1) (layers *.Cu *.Mask) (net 4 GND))
  (pad 2 thru_hole oval (at 0 2.54 90) (size 1.7 1.7) (drill 1) (layers *.Cu *.Mask) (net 56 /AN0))
  (pad 3 thru_hole oval (at 0 5.08 90) (size 1.7 1.7) (drill 1) (layers *.Cu *.Mask) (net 8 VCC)))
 (gr_line (start 39.497 49.022) (end 39.8145 49.022) (layer Edge.Cuts) (width 0.05))
 (gr_line (start 39.497 101.6) (end 39.497 49.022) (layer Edge.Cuts) (width 0.05))
 (gr_line (start 49.2125 49.022) (end 39.8145 49.022) (layer Edge.Cuts) (width 0.05))
 (gr_line (start 49.2125 49.022) (end 52.0065 45.72) (layer Edge.Cuts) (width 0.05))
 (gr_line (start 58.8645 49.022) (end 56.3245 45.72) (layer Edge.Cuts) (width 0.05))
 (gr_line (start 56.3245 45.72) (end 52.0065 45.72) (layer Edge.Cuts) (width 0.05))
 (gr_line (start 93.6625 49.022) (end 58.8645 49.022) (layer Edge.Cuts) (width 0.05))
 (gr_line (start 96.52 45.72) (end 93.6625 49.022) (layer Edge.Cuts) (width 0.05))
 (gr_line (start 100.076 45.72) (end 96.52 45.72) (layer Edge.Cuts) (width 0.05))
 (gr_line (start 102.87 49.022) (end 100.076 45.72) (layer Edge.Cuts) (width 0.05))
 (gr_line (start 111.125 49.022) (end 102.87 49.022) (layer Edge.Cuts) (width 0.05))
 (gr_line (start 56.9595 106.172) (end 50.038 106.172) (layer Edge.Cuts) (width 0.05))
 (gr_line (start 60.5155 101.6) (end 56.9595 106.172) (layer Edge.Cuts) (width 0.05))
 (gr_line (start 46.99 101.6) (end 39.497 101.6) (layer Edge.Cuts) (width 0.05))
 (gr_line (start 50.038 106.172) (end 46.99 101.6) (layer Edge.Cuts) (width 0.05))
 (gr_line (start 91.694 101.6) (end 60.5155 101.6) (layer Edge.Cuts) (width 0.05))
 (gr_line (start 94.996 106.172) (end 91.694 101.6) (layer Edge.Cuts) (width 0.05))
 (gr_line (start 101.6 106.172) (end 94.996 106.172) (layer Edge.Cuts) (width 0.05))
 (gr_line (start 104.3305 101.6) (end 101.6 106.172) (layer Edge.Cuts) (width 0.05))
 (gr_line (start 111.125 101.6) (end 104.3305 101.6) (layer Edge.Cuts) (width 0.05))
 (gr_line (start 111.125 49.022) (end 111.125 101.6) (layer Edge.Cuts) (width 0.05))
 (segment (start 54.951 78.74) (end 54.951 79.081) (width 0.254) (layer F.Cu) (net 8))
 (segment (start 58.2955 78.74) (end 54.951 78.74) (width 0.254) (layer F.Cu) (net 8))
 (segment (start 58.359 84.455) (end 55.179 84.455) (width 0.254) (layer F.Cu) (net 8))
 (segment (start 97.5995 79.9465) (end 94.234 83.312) (width 0.508) (layer F.Cu) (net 8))
 (segment (start 80.391 83.312) (end 77.2795 80.2005) (width 0.508) (layer F.Cu) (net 8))
 (segment (start 94.234 83.312) (end 80.391 83.312) (width 0.508) (layer F.Cu) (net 8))
 (segment (start 81.7245 84.6455) (end 80.391 83.312) (width 0.508) (layer F.Cu) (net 8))
 (segment (start 81.7245 90.9955) (end 81.7245 84.6455) (width 0.508) (layer F.Cu) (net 8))
 (segment (start 63.5635 68.8975) (end 65.913 66.548) (width 0.508) (layer F.Cu) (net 8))
 (segment (start 60.6425 68.8975) (end 63.5635 68.8975) (width 0.508) (layer F.Cu) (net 8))
 (segment (start 43.8785 69.9135) (end 42.8625 69.9135) (width 0.508) (layer F.Cu) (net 8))
 (segment (start 42.8625 69.9135) (end 41.656 71.12) (width 0.508) (layer F.Cu) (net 8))
 (segment (start 41.656 71.12) (end 41.656 98.044) (width 0.508) (layer F.Cu) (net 8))
 (segment (start 41.656 98.044) (end 43.434 99.822) (width 0.508) (layer F.Cu) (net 8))
 (segment (start 49.022 99.822) (end 53.594 95.25) (width 0.508) (layer F.Cu) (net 8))
 (segment (start 43.434 99.822) (end 49.022 99.822) (width 0.508) (layer F.Cu) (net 8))
 (segment (start 53.594 95.25) (end 56.134 95.25) (width 0.508) (layer F.Cu) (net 8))
 (segment (start 56.134 95.25) (end 58.674 95.25) (width 0.508) (layer F.Cu) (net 8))
 (segment (start 56.134 85.41) (end 55.179 84.455) (width 0.254) (layer F.Cu) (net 8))
 (segment (start 56.134 95.25) (end 56.134 85.41) (width 0.254) (layer F.Cu) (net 8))
 (segment (start 54.951 84.227) (end 55.179 84.455) (width 0.254) (layer F.Cu) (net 8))
 (segment (start 54.951 78.74) (end 54.951 84.227) (width 0.254) (layer F.Cu) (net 8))
 (segment (start 72.771 89.662) (end 74.1045 90.9955) (width 0.254) (layer B.Cu) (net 47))
 (segment (start 65.532 89.662) (end 72.771 89.662) (width 0.254) (layer B.Cu) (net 47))
 (segment (start 64.77 90.424) (end 65.532 89.662) (width 0.254) (layer B.Cu) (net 47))
 (segment (start 64.77 94.234) (end 64.77 90.424) (width 0.254) (layer B.Cu) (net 47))
 (segment (start 61.1505 97.8535) (end 64.77 94.234) (width 0.254) (layer B.Cu) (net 47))
 (segment (start 46.4185 97.8535) (end 61.1505 97.8535) (width 0.254) (layer B.Cu) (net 47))
 (segment (start 67.661501 92.358499) (end 67.661501 94.100461) (width 0.254) (layer B.Cu) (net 49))
 (segment (start 67.661501 94.100461) (end 62.955962 98.806) (width 0.254) (layer B.Cu) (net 49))
 (segment (start 69.0245 90.9955) (end 67.661501 92.358499) (width 0.254) (layer B.Cu) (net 49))
 (segment (start 62.955962 98.806) (end 62.955962 98.842038) (width 0.254) (layer B.Cu) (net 49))
 (segment (start 62.955962 98.842038) (end 62.23 99.568) (width 0.254) (layer B.Cu) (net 49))
 (segment (start 62.23 99.568) (end 45.72 99.568) (width 0.254) (layer B.Cu) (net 49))
 (segment (start 45.212 99.089499) (end 45.212 96.295499) (width 0.254) (layer B.Cu) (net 49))
 (segment (start 45.72 99.568) (end 45.241499 99.089499) (width 0.254) (layer B.Cu) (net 49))
 (segment (start 46.223498 95.3135) (end 46.4185 95.3135) (width 0.254) (layer B.Cu) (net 49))
 (segment (start 45.241499 96.295499) (end 46.223498 95.3135) (width 0.254) (layer B.Cu) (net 49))
 (segment (start 106.299 73.66) (end 107.5055 72.4535) (width 0.254) (layer B.Cu) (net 24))
 (segment (start 90.424 73.7235) (end 106.299 73.7235) (width 0.254) (layer B.Cu) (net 24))
 (segment (start 76.6445 87.4395) (end 90.424 73.66) (width 0.254) (layer B.Cu) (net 24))
 (segment (start 76.6445 90.9955) (end 76.6445 87.4395) (width 0.254) (layer B.Cu) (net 24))
 (segment (start 106.299 83.82) (end 107.5055 82.6135) (width 0.254) (layer B.Cu) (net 30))
 (segment (start 102.108 83.82) (end 106.299 83.82) (width 0.254) (layer B.Cu) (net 30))
 (segment (start 90.424 95.504) (end 102.108 83.82) (width 0.254) (layer B.Cu) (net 30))
 (segment (start 73.66 95.504) (end 90.424 95.504) (width 0.254) (layer B.Cu) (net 30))
 (segment (start 72.898 94.742) (end 73.66 95.504) (width 0.254) (layer B.Cu) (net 30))
 (segment (start 72.898 92.329) (end 72.898 94.742) (width 0.254) (layer B.Cu) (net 30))
 (segment (start 71.5645 90.9955) (end 72.898 92.329) (width 0.254) (layer B.Cu) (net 30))
 (segment (start 74.7395 80.2005) (end 73.406 81.534) (width 0.254) (layer B.Cu) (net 56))
 (segment (start 73.406 81.534) (end 52.324 81.534) (width 0.254) (layer B.Cu) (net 56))
 (segment (start 50.067499 83.790501) (end 45.241499 83.790501) (width 0.254) (layer B.Cu) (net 56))
 (segment (start 52.324 81.534) (end 50.067499 83.790501) (width 0.254) (layer B.Cu) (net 56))
 (segment (start 45.241499 83.790501) (end 44.577 84.455) (width 0.254) (layer B.Cu) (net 56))
 (segment (start 44.577 84.455) (end 43.8785 85.1535) (width 0.254) (layer B.Cu) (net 56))
 (segment (start 108.070461 81.436499) (end 109.474 82.840038) (width 0.254) (layer B.Cu) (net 5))
 (segment (start 91.476038 81.3435) (end 108.077 81.3435) (width 0.254) (layer B.Cu) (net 5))
 (segment (start 89.9795 79.9465) (end 91.469499 81.436499) (width 0.254) (layer B.Cu) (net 5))
 (segment (start 109.474 90.805) (end 107.5055 92.7735) (width 0.254) (layer B.Cu) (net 5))
 (segment (start 109.474 82.840038) (end 109.474 90.805) (width 0.254) (layer B.Cu) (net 5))
 (segment (start 107.569 77.597) (end 107.5055 77.5335) (width 0.25) (layer B.Cu) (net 1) (status 30))
 (segment (start 107.5055 77.4065) (end 107.5055 77.5335) (width 0.254) (layer B.Cu) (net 1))
 (segment (start 106.172 76.2) (end 107.5055 77.5335) (width 0.254) (layer B.Cu) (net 1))
 (segment (start 103.886 76.2635) (end 106.172 76.2635) (width 0.254) (layer B.Cu) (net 1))
 (segment (start 102.6795 77.4065) (end 103.886 76.2) (width 0.254) (layer B.Cu) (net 1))
 (segment (start 97.5995 77.4065) (end 102.6795 77.4065) (width 0.254) (layer B.Cu) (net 1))
 (segment (start 58.1025 68.8975) (end 58.1025 70.231) (width 0.254) (layer B.Cu) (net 13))
 (segment (start 58.1025 70.231) (end 58.7375 70.866) (width 0.254) (layer B.Cu) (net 13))
 (segment (start 69.215 70.866) (end 73.533 66.548) (width 0.254) (layer B.Cu) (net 13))
 (segment (start 58.7375 70.866) (end 69.215 70.866) (width 0.254) (layer B.Cu) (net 13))
 (segment (start 106.328499 56.036499) (end 107.5055 57.2135) (width 0.254) (layer B.Cu) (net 13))
 (segment (start 84.044501 55.9435) (end 106.328499 55.9435) (width 0.254) (layer B.Cu) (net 13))
 (segment (start 73.533 66.548) (end 84.044501 56.036499) (width 0.254) (layer B.Cu) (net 13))
 (segment (start 55.5625 68.8975) (end 57.277 67.183) (width 0.254) (layer B.Cu) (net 11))
 (segment (start 57.277 67.183) (end 61.341 67.183) (width 0.254) (layer B.Cu) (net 11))
 (segment (start 61.341 67.183) (end 63.9445 69.7865) (width 0.254) (layer B.Cu) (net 11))
 (segment (start 67.7545 69.7865) (end 70.993 66.548) (width 0.254) (layer B.Cu) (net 11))
 (segment (start 63.9445 69.7865) (end 67.7545 69.7865) (width 0.254) (layer B.Cu) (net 11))
 (segment (start 106.328499 53.496499) (end 107.5055 54.6735) (width 0.254) (layer B.Cu) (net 11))
 (segment (start 84.044501 53.4035) (end 106.328499 53.4035) (width 0.254) (layer B.Cu) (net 11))
 (segment (start 70.993 66.548) (end 84.044501 53.496499) (width 0.254) (layer B.Cu) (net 11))
 (segment (start 55.666 76.2) (end 53.126 78.74) (width 0.254) (layer F.Cu) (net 7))
 (segment (start 83.312 76.2) (end 55.666 76.2) (width 0.254) (layer F.Cu) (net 7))
 (segment (start 95.0595 79.9465) (end 93.853 78.74) (width 0.254) (layer F.Cu) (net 7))
 (segment (start 93.853 78.74) (end 85.852 78.74) (width 0.254) (layer F.Cu) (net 7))
 (segment (start 85.852 78.74) (end 83.312 76.2) (width 0.254) (layer F.Cu) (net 7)))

